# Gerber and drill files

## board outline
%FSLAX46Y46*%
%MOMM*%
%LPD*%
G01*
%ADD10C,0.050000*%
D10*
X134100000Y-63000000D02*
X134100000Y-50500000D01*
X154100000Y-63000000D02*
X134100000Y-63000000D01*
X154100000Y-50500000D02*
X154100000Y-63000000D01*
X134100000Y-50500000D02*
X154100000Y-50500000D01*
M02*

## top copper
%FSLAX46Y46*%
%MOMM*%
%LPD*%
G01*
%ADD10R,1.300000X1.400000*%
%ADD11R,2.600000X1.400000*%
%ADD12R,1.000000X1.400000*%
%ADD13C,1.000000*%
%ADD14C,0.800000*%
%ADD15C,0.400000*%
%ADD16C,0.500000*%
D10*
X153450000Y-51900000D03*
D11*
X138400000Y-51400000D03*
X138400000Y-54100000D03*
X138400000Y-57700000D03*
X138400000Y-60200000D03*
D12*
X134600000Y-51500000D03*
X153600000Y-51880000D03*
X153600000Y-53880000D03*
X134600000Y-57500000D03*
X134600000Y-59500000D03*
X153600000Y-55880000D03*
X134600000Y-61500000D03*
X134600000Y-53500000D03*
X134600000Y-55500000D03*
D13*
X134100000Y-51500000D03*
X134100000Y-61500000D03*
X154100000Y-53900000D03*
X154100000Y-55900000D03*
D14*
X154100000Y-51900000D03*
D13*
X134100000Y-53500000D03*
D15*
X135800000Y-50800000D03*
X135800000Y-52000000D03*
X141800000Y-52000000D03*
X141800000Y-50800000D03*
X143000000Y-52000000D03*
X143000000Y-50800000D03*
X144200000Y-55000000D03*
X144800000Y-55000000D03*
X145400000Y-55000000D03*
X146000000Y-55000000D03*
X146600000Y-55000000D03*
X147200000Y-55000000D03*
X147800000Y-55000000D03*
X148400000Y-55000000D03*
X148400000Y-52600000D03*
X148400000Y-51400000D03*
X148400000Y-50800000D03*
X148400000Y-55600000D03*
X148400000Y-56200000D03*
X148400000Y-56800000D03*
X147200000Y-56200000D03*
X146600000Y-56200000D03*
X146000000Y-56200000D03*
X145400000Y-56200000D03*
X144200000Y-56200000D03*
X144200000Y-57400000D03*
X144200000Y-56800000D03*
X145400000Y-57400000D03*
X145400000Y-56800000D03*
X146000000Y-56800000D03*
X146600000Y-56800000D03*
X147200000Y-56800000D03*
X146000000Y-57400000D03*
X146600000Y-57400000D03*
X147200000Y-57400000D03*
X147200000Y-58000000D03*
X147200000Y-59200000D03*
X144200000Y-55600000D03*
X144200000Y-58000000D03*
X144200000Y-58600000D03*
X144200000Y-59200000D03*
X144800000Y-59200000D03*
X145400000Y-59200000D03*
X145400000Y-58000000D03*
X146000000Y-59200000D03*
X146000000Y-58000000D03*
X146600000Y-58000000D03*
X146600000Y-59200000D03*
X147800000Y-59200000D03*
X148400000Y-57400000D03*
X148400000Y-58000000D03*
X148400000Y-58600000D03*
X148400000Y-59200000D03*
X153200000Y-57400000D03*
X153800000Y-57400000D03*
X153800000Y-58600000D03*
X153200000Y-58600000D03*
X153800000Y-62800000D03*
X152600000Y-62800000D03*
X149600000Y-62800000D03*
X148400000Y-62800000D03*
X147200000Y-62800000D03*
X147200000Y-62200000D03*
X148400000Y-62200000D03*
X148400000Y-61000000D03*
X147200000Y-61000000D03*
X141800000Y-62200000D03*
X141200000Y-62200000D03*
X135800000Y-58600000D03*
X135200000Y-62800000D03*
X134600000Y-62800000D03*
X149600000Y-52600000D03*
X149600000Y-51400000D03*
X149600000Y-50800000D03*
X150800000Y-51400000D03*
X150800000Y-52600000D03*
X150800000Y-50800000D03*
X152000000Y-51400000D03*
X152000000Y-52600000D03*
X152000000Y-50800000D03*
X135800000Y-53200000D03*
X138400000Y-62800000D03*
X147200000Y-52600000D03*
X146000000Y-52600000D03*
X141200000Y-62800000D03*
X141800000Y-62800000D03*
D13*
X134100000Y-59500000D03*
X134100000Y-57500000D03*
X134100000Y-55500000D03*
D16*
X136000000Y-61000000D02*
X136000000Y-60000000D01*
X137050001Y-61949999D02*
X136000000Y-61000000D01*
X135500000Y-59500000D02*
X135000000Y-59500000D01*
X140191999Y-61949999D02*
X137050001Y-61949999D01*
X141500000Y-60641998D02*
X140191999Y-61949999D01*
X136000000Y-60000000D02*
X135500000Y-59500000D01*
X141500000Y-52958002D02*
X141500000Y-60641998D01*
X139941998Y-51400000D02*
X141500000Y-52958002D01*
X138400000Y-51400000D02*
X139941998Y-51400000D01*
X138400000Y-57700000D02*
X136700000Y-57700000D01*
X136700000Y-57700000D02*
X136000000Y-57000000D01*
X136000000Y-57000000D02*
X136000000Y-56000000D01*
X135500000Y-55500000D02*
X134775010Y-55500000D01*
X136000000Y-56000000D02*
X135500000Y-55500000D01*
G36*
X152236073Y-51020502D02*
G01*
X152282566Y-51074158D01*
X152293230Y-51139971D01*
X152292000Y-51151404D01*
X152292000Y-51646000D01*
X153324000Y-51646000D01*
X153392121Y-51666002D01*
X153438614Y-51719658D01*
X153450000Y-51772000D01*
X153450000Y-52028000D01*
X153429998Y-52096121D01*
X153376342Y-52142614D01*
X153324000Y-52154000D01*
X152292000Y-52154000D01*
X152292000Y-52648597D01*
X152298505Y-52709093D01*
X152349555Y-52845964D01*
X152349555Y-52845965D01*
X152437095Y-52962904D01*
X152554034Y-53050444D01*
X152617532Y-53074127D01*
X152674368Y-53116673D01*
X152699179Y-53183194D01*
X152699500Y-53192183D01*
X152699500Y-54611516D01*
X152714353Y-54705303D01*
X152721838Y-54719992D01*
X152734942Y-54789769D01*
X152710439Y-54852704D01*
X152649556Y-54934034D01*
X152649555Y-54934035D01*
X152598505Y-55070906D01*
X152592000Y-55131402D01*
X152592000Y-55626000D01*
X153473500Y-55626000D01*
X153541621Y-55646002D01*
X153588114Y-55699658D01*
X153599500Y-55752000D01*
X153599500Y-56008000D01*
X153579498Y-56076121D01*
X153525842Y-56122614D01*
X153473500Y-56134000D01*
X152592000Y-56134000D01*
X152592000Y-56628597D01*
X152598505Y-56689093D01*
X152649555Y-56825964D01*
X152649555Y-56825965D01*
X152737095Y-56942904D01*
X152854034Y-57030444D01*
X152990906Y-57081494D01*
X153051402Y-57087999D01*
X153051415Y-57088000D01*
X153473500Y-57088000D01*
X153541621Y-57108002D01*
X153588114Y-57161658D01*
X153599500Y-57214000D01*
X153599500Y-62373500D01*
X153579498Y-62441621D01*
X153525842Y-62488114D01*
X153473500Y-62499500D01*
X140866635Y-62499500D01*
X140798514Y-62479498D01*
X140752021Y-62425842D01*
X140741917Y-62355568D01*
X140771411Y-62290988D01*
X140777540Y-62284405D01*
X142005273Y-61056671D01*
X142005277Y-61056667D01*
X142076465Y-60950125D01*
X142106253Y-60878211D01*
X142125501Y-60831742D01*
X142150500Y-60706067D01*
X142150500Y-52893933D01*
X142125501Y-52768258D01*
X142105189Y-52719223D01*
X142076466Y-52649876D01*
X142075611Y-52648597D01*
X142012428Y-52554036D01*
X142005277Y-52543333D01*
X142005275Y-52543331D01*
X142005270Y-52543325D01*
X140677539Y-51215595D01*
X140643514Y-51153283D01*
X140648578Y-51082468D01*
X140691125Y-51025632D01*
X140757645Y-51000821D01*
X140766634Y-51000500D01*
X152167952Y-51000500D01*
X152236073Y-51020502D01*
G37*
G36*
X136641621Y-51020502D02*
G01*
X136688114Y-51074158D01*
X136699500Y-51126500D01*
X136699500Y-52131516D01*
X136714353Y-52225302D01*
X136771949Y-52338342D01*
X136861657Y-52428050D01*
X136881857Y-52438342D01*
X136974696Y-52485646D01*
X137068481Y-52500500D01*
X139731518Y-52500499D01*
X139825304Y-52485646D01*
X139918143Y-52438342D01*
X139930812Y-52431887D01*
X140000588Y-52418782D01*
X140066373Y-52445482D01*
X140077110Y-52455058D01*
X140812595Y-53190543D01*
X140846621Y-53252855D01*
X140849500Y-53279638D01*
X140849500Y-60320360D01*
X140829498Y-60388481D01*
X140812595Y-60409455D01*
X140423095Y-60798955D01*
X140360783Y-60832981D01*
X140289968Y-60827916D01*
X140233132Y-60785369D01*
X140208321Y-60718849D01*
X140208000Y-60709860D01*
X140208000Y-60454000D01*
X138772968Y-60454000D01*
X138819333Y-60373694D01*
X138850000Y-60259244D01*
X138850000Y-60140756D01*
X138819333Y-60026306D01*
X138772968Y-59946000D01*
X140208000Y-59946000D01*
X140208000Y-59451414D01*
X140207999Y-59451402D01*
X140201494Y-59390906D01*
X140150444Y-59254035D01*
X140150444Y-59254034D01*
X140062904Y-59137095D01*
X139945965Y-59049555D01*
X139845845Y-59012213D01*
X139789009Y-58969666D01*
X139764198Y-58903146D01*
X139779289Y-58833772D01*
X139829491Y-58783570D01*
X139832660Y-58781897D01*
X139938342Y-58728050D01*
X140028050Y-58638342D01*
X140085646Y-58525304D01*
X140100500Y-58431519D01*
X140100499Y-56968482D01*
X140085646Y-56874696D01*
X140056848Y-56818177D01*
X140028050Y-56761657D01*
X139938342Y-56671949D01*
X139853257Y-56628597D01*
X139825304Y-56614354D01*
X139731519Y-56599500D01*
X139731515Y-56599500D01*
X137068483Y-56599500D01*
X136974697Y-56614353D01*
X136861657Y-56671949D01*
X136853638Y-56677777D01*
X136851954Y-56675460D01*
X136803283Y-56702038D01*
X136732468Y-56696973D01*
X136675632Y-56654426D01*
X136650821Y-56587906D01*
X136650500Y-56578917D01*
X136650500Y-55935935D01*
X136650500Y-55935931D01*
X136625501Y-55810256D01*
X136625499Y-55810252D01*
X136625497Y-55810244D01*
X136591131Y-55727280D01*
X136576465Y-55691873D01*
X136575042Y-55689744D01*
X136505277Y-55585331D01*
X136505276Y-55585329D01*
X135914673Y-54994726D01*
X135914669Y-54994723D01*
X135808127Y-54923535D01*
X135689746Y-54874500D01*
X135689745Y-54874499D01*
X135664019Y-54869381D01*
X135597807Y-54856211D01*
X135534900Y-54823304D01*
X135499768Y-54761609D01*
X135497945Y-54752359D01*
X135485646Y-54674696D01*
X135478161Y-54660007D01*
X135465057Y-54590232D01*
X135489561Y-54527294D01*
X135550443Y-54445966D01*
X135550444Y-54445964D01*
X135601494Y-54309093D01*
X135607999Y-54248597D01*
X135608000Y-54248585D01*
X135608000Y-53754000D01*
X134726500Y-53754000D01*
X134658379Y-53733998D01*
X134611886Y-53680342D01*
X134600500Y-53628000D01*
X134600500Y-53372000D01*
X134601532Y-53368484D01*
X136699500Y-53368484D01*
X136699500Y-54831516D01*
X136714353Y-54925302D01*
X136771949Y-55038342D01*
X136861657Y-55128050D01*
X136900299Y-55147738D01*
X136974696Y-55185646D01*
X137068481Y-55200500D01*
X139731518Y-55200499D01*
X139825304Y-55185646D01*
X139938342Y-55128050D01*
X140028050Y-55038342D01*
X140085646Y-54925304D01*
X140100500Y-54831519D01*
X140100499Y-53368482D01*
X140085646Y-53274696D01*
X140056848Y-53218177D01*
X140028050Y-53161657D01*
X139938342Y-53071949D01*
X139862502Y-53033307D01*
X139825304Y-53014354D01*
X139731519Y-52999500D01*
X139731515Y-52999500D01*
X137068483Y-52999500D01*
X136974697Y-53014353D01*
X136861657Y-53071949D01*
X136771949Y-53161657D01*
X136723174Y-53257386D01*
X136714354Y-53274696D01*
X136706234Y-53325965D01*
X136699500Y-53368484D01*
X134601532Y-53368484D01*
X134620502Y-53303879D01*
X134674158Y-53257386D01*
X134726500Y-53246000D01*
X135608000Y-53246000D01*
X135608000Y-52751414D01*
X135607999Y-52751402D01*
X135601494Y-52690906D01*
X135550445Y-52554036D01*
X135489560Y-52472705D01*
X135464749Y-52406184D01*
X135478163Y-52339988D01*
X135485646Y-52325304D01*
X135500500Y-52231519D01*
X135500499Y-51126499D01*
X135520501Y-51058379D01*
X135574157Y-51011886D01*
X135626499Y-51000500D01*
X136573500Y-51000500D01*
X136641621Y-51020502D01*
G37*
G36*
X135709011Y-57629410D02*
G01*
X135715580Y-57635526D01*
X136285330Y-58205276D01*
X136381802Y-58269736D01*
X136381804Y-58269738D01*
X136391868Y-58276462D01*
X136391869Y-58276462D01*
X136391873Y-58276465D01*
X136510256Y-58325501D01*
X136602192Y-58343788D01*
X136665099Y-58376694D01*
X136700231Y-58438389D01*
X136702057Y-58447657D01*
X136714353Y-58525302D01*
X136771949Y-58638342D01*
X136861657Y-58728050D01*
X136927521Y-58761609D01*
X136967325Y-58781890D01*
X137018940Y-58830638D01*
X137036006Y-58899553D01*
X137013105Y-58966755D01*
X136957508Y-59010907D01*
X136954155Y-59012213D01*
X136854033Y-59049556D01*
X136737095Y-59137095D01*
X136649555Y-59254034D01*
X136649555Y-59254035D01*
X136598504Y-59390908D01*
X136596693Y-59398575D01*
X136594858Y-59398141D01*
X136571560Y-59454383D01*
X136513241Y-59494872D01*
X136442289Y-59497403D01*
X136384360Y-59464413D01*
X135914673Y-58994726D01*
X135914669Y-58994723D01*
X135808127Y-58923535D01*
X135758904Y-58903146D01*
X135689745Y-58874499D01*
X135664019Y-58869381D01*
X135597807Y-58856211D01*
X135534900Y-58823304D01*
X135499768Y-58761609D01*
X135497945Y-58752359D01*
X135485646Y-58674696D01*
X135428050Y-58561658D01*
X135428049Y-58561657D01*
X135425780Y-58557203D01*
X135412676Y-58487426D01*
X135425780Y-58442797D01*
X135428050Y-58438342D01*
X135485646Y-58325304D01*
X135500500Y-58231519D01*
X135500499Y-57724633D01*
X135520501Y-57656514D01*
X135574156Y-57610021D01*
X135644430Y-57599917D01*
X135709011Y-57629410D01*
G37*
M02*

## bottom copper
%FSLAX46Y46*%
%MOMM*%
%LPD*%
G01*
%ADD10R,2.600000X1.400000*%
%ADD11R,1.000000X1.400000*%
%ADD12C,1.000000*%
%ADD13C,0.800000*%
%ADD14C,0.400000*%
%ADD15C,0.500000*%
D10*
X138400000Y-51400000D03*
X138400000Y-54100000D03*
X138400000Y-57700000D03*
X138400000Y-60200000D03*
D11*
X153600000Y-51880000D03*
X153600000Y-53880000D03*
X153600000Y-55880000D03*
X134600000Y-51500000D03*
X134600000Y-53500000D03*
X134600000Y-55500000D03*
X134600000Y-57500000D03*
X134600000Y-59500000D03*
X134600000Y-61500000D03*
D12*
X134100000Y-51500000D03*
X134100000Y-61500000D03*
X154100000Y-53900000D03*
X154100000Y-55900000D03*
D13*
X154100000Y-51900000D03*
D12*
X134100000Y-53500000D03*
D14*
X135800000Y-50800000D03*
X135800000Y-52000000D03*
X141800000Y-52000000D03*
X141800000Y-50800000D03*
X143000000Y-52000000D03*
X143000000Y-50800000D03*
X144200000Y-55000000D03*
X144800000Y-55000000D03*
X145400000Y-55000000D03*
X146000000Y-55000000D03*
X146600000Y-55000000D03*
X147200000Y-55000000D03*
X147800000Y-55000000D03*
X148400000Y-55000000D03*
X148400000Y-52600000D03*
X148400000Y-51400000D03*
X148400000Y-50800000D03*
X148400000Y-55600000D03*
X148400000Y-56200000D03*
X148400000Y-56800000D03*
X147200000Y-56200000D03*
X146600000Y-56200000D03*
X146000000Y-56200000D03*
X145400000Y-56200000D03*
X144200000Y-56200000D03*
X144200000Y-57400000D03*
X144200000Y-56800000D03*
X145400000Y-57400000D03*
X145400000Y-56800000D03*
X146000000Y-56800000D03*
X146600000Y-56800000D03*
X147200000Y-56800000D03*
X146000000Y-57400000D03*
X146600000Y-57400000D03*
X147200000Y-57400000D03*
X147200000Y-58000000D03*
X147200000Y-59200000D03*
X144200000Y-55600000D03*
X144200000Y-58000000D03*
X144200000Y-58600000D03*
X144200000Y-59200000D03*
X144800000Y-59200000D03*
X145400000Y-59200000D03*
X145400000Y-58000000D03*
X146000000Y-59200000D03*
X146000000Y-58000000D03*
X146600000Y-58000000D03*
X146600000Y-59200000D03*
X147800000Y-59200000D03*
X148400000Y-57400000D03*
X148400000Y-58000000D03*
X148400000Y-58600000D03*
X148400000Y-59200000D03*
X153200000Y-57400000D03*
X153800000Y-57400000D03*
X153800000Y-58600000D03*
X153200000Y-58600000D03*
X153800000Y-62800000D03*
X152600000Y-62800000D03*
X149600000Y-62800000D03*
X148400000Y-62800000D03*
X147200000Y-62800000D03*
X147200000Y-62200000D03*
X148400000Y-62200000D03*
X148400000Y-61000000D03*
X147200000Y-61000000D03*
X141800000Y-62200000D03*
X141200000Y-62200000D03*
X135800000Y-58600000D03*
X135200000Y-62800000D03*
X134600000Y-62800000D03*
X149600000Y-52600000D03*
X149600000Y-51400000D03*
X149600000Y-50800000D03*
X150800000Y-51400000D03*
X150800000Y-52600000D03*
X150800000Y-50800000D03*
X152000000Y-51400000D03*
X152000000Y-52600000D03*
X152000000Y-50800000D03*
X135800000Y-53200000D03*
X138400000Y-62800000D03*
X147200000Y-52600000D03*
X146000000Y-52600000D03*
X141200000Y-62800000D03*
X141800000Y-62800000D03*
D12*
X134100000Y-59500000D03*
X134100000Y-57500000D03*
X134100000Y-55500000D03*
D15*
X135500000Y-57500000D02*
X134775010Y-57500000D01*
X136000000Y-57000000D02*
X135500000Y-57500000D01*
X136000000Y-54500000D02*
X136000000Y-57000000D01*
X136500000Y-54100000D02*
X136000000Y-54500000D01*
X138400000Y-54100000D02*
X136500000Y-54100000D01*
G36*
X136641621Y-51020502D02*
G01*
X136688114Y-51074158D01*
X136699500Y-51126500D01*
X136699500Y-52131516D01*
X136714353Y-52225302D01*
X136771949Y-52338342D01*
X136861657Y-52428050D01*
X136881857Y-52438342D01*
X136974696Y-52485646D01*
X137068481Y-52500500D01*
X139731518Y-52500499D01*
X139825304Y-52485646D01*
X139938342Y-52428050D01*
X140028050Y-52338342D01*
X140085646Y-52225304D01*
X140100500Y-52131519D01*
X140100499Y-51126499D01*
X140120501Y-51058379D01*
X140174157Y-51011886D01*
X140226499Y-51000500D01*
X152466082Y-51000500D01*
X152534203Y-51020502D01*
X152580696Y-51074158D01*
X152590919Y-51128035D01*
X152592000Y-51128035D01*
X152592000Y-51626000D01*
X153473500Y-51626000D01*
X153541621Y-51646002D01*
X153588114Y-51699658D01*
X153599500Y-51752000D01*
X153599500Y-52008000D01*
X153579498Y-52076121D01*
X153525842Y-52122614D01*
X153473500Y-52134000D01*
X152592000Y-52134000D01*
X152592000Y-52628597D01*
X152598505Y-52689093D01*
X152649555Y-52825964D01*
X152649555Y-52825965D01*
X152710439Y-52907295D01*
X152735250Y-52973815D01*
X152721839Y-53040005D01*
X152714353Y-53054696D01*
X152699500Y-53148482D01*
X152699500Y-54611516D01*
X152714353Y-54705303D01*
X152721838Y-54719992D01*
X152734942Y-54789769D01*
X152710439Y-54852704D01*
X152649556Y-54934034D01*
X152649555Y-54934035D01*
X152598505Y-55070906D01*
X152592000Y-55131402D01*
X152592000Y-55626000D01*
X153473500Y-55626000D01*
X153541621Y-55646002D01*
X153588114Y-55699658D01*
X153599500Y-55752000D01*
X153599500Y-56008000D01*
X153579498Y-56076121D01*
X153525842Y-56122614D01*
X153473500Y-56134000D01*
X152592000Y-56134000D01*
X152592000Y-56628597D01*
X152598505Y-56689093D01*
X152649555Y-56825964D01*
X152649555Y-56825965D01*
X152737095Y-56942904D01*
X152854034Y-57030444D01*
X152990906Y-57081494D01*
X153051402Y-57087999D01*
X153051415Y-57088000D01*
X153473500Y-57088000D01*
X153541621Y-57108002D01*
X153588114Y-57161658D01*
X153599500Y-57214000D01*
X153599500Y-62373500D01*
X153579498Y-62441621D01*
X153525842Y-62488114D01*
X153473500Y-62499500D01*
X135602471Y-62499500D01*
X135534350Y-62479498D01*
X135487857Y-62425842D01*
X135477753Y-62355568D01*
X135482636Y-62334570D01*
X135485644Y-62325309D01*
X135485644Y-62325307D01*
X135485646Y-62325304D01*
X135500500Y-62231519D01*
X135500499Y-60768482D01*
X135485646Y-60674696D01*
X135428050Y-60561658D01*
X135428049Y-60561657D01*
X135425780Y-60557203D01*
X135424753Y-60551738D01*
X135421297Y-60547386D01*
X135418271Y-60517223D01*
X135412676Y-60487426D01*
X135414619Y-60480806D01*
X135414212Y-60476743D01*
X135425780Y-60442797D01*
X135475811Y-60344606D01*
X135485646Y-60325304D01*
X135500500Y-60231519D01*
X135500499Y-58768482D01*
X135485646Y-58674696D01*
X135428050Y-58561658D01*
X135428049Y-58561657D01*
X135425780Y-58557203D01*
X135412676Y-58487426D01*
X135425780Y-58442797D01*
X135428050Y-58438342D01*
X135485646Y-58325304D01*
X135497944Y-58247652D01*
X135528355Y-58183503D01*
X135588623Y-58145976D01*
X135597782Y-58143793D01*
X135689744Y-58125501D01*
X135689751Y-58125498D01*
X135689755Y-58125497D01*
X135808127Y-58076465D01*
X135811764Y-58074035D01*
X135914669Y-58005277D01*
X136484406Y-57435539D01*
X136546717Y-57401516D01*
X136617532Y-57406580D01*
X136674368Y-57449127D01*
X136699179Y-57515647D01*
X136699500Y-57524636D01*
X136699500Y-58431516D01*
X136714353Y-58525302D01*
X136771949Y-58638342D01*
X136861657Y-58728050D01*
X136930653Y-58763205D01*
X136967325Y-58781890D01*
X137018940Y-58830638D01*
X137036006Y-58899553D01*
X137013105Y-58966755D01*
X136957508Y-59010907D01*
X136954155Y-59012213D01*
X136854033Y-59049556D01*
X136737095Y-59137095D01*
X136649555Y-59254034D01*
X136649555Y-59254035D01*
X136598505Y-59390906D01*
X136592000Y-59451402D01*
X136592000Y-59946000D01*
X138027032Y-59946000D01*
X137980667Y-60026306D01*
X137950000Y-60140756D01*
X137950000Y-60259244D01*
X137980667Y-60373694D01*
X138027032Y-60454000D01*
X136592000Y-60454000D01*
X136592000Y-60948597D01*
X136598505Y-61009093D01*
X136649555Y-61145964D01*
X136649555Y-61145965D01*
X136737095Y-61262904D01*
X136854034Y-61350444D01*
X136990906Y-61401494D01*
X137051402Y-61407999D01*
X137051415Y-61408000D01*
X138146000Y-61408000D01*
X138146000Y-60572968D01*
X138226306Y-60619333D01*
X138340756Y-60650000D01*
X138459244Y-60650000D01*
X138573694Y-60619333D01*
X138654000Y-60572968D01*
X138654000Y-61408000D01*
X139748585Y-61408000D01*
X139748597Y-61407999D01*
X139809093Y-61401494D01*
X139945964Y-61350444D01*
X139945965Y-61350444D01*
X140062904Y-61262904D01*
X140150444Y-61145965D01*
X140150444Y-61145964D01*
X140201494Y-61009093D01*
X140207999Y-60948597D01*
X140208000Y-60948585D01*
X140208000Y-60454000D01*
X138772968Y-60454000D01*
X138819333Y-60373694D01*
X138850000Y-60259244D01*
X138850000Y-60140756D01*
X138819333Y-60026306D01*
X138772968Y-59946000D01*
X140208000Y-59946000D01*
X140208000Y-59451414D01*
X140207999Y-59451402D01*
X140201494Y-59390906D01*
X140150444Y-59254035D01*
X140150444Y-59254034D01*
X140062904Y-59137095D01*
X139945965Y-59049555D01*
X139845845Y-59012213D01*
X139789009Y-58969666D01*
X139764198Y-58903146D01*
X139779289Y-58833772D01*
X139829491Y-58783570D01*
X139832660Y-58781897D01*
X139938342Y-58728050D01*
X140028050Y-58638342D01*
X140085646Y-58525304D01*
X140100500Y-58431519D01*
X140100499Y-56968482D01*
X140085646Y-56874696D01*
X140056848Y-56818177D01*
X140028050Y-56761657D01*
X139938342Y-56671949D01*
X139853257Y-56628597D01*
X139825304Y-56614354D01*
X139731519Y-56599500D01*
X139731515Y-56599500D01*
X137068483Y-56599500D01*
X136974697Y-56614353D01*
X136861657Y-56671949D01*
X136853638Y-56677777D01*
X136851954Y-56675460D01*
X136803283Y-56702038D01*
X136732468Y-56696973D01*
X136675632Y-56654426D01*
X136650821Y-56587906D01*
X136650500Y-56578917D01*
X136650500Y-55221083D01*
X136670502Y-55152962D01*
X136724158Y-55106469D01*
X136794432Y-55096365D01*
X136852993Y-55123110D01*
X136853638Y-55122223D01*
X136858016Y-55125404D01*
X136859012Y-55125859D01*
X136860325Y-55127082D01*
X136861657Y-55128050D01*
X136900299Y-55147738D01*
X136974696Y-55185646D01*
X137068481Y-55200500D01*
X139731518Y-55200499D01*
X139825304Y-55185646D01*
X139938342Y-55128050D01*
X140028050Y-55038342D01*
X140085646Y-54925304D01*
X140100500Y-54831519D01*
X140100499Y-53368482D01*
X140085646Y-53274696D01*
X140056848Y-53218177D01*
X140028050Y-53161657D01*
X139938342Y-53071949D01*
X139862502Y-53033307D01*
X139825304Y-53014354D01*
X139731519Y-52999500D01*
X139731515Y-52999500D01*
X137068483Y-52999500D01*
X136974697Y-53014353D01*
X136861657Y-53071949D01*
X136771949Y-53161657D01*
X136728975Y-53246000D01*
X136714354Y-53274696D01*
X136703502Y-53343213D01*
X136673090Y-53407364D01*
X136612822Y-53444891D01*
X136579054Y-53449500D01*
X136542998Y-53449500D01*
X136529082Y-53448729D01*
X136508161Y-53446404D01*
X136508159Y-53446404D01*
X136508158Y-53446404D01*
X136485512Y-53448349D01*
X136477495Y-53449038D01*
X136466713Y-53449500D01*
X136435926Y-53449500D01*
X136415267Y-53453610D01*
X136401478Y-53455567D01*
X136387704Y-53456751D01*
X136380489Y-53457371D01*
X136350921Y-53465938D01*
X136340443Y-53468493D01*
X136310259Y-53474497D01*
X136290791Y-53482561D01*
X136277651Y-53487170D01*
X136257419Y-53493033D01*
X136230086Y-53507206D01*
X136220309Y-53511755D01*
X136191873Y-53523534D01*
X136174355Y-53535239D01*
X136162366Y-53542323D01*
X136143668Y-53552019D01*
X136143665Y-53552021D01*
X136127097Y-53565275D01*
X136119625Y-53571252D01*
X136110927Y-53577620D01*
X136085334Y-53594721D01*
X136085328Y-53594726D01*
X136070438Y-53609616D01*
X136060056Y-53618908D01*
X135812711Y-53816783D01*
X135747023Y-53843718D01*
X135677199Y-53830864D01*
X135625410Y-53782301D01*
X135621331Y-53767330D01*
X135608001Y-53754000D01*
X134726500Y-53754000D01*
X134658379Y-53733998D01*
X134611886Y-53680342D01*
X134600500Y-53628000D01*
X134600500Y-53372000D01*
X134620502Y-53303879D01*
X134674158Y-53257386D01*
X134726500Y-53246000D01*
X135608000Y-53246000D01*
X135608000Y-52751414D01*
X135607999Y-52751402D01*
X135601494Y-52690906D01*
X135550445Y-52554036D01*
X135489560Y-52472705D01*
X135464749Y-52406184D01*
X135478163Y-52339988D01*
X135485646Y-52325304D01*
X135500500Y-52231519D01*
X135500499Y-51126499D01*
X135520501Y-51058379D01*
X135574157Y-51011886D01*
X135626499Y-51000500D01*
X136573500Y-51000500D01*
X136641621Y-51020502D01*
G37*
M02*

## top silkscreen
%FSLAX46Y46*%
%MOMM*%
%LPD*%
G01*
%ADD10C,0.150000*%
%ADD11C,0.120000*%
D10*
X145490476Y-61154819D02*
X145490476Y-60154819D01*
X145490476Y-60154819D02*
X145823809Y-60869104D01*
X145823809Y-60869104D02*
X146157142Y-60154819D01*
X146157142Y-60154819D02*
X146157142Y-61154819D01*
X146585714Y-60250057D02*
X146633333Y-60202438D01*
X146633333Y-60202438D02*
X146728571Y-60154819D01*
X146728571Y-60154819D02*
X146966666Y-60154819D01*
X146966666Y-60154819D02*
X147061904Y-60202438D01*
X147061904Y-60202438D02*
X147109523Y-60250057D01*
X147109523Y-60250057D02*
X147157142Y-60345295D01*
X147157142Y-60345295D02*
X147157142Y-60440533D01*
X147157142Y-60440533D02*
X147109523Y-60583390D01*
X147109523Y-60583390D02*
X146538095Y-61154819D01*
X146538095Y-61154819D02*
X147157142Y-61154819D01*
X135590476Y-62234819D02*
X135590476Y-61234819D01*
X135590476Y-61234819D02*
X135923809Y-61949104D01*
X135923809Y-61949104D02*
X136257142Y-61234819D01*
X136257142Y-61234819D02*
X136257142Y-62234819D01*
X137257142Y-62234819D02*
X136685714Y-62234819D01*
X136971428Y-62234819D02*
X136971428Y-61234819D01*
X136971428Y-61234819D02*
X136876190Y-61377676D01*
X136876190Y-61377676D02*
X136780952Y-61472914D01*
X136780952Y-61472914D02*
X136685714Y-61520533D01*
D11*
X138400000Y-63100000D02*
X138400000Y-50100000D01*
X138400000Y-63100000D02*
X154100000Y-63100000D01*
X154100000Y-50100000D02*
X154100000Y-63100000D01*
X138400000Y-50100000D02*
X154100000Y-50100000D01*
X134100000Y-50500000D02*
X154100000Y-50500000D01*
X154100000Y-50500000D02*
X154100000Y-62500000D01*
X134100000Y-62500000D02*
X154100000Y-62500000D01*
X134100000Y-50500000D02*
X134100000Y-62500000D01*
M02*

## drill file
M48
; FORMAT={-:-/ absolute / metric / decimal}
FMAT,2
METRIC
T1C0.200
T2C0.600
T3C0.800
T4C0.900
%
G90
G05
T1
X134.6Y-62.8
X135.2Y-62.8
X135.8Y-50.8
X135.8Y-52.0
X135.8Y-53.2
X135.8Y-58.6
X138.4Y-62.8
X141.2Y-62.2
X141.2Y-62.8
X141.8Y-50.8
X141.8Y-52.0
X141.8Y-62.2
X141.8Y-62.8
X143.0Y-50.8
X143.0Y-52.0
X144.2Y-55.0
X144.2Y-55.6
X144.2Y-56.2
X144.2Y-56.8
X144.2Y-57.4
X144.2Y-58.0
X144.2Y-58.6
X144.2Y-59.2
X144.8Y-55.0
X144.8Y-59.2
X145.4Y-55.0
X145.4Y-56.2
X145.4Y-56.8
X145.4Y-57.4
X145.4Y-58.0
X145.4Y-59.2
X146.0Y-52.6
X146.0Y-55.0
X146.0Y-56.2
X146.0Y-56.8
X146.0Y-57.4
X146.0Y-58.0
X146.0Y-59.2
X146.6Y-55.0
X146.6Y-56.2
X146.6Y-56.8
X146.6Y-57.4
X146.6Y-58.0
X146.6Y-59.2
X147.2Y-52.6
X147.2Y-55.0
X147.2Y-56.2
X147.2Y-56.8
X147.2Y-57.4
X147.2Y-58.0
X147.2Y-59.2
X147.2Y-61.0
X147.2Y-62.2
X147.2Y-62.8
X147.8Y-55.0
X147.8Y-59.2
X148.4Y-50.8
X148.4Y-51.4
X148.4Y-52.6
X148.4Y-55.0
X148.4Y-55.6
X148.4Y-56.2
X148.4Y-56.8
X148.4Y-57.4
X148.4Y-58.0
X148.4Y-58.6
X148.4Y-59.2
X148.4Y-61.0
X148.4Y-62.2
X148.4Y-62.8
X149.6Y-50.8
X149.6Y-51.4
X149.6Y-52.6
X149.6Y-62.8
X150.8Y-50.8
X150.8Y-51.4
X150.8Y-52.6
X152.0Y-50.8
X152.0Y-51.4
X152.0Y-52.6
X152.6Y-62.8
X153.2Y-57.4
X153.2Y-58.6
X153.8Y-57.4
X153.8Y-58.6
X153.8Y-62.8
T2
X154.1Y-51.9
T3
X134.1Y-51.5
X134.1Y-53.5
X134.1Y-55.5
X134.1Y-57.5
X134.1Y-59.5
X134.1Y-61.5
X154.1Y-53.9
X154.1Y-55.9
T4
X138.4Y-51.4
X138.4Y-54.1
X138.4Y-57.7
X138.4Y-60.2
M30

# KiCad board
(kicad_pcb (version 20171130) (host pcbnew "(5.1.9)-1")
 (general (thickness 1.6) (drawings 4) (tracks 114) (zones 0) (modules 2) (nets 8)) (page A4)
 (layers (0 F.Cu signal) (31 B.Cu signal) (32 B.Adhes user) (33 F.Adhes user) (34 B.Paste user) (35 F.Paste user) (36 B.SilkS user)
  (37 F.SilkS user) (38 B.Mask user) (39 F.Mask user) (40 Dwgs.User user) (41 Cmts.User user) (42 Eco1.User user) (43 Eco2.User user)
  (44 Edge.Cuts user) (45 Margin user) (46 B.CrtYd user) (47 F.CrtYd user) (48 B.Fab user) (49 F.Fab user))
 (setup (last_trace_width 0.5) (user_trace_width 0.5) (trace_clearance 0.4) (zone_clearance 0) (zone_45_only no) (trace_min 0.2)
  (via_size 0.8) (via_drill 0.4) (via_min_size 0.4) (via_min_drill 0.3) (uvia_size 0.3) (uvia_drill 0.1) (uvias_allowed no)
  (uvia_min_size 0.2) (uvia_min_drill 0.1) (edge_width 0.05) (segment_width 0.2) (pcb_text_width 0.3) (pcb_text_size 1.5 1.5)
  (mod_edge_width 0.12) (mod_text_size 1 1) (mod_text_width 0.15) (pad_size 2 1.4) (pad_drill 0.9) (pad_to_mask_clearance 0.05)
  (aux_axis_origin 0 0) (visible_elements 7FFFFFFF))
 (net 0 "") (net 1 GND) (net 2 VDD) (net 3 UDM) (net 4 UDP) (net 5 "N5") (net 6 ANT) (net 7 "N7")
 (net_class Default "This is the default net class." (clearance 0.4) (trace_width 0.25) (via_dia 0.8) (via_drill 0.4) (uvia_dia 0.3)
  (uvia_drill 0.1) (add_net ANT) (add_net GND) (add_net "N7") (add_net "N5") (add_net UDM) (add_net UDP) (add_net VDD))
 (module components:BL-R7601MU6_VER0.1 (layer F.Cu) (at 138.4 50.1)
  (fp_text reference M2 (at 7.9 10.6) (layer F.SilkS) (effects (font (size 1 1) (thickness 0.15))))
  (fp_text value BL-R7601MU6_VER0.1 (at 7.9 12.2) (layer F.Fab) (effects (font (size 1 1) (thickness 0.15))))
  (fp_line (start 0 13) (end 0 0) (layer F.SilkS) (width 0.12))
  (fp_line (start 0 13) (end 15.7 13) (layer F.SilkS) (width 0.12))
  (fp_line (start 15.7 0) (end 15.7 13) (layer F.SilkS) (width 0.12))
  (fp_line (start 0 0) (end 15.7 0) (layer F.SilkS) (width 0.12))
  (pad 5 smd rect (at 15.7 1.8) (size 1.3 1.4) (drill (offset -0.65 0)) (layers F.Cu F.Paste F.Mask) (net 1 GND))
  (pad 4 thru_hole rect (at 0 1.3) (size 2.6 1.4) (drill 0.9) (layers *.Cu *.Mask) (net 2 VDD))
  (pad 3 thru_hole rect (at 0 4) (size 2.6 1.4) (drill 0.9) (layers *.Cu *.Mask) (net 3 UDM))
  (pad 2 thru_hole rect (at 0 7.6) (size 2.6 1.4) (drill 0.9) (layers *.Cu *.Mask) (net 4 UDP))
  (pad 1 thru_hole rect (at 0 10.1) (size 2.6 1.4) (drill 0.9) (layers *.Cu *.Mask) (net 1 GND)))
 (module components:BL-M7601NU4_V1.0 (layer F.Cu) (at 134.1 50.5)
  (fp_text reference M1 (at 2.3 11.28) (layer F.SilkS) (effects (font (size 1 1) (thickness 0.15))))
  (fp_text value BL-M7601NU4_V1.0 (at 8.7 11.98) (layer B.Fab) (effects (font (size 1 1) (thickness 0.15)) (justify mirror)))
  (fp_line (start 0 0) (end 20 0) (layer F.SilkS) (width 0.12))
  (fp_line (start 20 0) (end 20 12) (layer F.SilkS) (width 0.12))
  (fp_line (start 0 12) (end 20 12) (layer F.SilkS) (width 0.12))
  (fp_line (start 0 0) (end 0 12) (layer F.SilkS) (width 0.12))
  (pad 6 smd rect (at 0 1) (size 1 1.4) (drill (offset 0.5 0)) (layers F.Cu F.Paste F.Mask) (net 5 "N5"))
  (pad 9 smd rect (at 20 1.38) (size 1 1.4) (drill (offset -0.5 0)) (layers F.Cu F.Paste F.Mask) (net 1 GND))
  (pad 8 smd rect (at 20 3.38) (size 1 1.4) (drill (offset -0.5 0)) (layers F.Cu F.Paste F.Mask) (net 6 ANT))
  (pad 3 smd rect (at 0 7) (size 1 1.4) (drill (offset 0.5 0)) (layers F.Cu F.Paste F.Mask) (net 3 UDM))
  (pad 2 smd rect (at 0 9) (size 1 1.4) (drill (offset 0.5 0)) (layers F.Cu F.Paste F.Mask) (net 2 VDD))
  (pad 7 smd rect (at 20 5.38) (size 1 1.4) (drill (offset -0.5 0)) (layers F.Cu F.Paste F.Mask) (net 1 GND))
  (pad 1 smd rect (at 0 11) (size 1 1.4) (drill (offset 0.5 0)) (layers F.Cu F.Paste F.Mask) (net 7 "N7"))
  (pad 5 smd rect (at 0 3) (size 1 1.4) (drill (offset 0.5 0)) (layers F.Cu F.Paste F.Mask) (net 1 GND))
  (pad 4 smd rect (at 0 5) (size 1 1.4) (drill (offset 0.5 0)) (layers F.Cu F.Paste F.Mask) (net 4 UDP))
  (pad 9 smd rect (at 20 1.38) (size 1 1.4) (drill (offset -0.5 0)) (layers B.Cu B.Paste B.Mask) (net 1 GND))
  (pad 8 smd rect (at 20 3.38) (size 1 1.4) (drill (offset -0.5 0)) (layers B.Cu B.Paste B.Mask) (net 6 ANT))
  (pad 7 smd rect (at 20 5.38) (size 1 1.4) (drill (offset -0.5 0)) (layers B.Cu B.Paste B.Mask) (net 1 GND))
  (pad 6 smd rect (at 0 1) (size 1 1.4) (drill (offset 0.5 0)) (layers B.Cu B.Paste B.Mask) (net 5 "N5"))
  (pad 5 smd rect (at 0 3) (size 1 1.4) (drill (offset 0.5 0)) (layers B.Cu B.Paste B.Mask) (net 1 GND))
  (pad 4 smd rect (at 0 5) (size 1 1.4) (drill (offset 0.5 0)) (layers B.Cu B.Paste B.Mask) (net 4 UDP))
  (pad 3 smd rect (at 0 7) (size 1 1.4) (drill (offset 0.5 0)) (layers B.Cu B.Paste B.Mask) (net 3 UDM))
  (pad 2 smd rect (at 0 9) (size 1 1.4) (drill (offset 0.5 0)) (layers B.Cu B.Paste B.Mask) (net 2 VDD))
  (pad 1 smd rect (at 0 11) (size 1 1.4) (drill (offset 0.5 0)) (layers B.Cu B.Paste B.Mask) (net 7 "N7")))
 (gr_line (start 134.1 63) (end 134.1 50.5) (layer Edge.Cuts) (width 0.05))
 (gr_line (start 154.1 63) (end 134.1 63) (layer Edge.Cuts) (width 0.05))
 (gr_line (start 154.1 50.5) (end 154.1 63) (layer Edge.Cuts) (width 0.05))
 (gr_line (start 134.1 50.5) (end 154.1 50.5) (layer Edge.Cuts) (width 0.05))
 (via (at 134.1 51.5) (size 1) (drill 0.8) (layers F.Cu B.Cu) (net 5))
 (via (at 134.1 61.5) (size 1) (drill 0.8) (layers F.Cu B.Cu) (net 7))
 (via (at 154.1 53.9) (size 1) (drill 0.8) (layers F.Cu B.Cu) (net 6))
 (via (at 154.1 55.9) (size 1) (drill 0.8) (layers F.Cu B.Cu) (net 1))
 (via (at 154.1 51.9) (size 0.8) (drill 0.6) (layers F.Cu B.Cu) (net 1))
 (via (at 134.1 53.5) (size 1) (drill 0.8) (layers F.Cu B.Cu) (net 1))
 (via (at 135.8 50.8) (size 0.4) (drill 0.2) (layers F.Cu B.Cu) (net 1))
 (via (at 135.8 52) (size 0.4) (drill 0.2) (layers F.Cu B.Cu) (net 1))
 (via (at 141.8 52) (size 0.4) (drill 0.2) (layers F.Cu B.Cu) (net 1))
 (via (at 141.8 50.8) (size 0.4) (drill 0.2) (layers F.Cu B.Cu) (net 1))
 (via (at 143 52) (size 0.4) (drill 0.2) (layers F.Cu B.Cu) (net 1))
 (via (at 143 50.8) (size 0.4) (drill 0.2) (layers F.Cu B.Cu) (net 1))
 (via (at 144.2 55) (size 0.4) (drill 0.2) (layers F.Cu B.Cu) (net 1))
 (via (at 144.8 55) (size 0.4) (drill 0.2) (layers F.Cu B.Cu) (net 1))
 (via (at 145.4 55) (size 0.4) (drill 0.2) (layers F.Cu B.Cu) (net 1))
 (via (at 146 55) (size 0.4) (drill 0.2) (layers F.Cu B.Cu) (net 1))
 (via (at 146.6 55) (size 0.4) (drill 0.2) (layers F.Cu B.Cu) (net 1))
 (via (at 147.2 55) (size 0.4) (drill 0.2) (layers F.Cu B.Cu) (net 1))
 (via (at 147.8 55) (size 0.4) (drill 0.2) (layers F.Cu B.Cu) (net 1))
 (via (at 148.4 55) (size 0.4) (drill 0.2) (layers F.Cu B.Cu) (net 1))
 (via (at 148.4 52.6) (size 0.4) (drill 0.2) (layers F.Cu B.Cu) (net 1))
 (via (at 148.4 51.4) (size 0.4) (drill 0.2) (layers F.Cu B.Cu) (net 1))
 (via (at 148.4 50.8) (size 0.4) (drill 0.2) (layers F.Cu B.Cu) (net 1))
 (via (at 148.4 55.6) (size 0.4) (drill 0.2) (layers F.Cu B.Cu) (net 1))
 (via (at 148.4 56.2) (size 0.4) (drill 0.2) (layers F.Cu B.Cu) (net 1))
 (via (at 148.4 56.8) (size 0.4) (drill 0.2) (layers F.Cu B.Cu) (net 1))
 (via (at 147.2 56.2) (size 0.4) (drill 0.2) (layers F.Cu B.Cu) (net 1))
 (via (at 146.6 56.2) (size 0.4) (drill 0.2) (layers F.Cu B.Cu) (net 1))
 (via (at 146 56.2) (size 0.4) (drill 0.2) (layers F.Cu B.Cu) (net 1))
 (via (at 145.4 56.2) (size 0.4) (drill 0.2) (layers F.Cu B.Cu) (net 1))
 (via (at 144.2 56.2) (size 0.4) (drill 0.2) (layers F.Cu B.Cu) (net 1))
 (via (at 144.2 57.4) (size 0.4) (drill 0.2) (layers F.Cu B.Cu) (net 1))
 (via (at 144.2 56.8) (size 0.4) (drill 0.2) (layers F.Cu B.Cu) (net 1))
 (via (at 145.4 57.4) (size 0.4) (drill 0.2) (layers F.Cu B.Cu) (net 1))
 (via (at 145.4 56.8) (size 0.4) (drill 0.2) (layers F.Cu B.Cu) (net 1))
 (via (at 146 56.8) (size 0.4) (drill 0.2) (layers F.Cu B.Cu) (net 1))
 (via (at 146.6 56.8) (size 0.4) (drill 0.2) (layers F.Cu B.Cu) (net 1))
 (via (at 147.2 56.8) (size 0.4) (drill 0.2) (layers F.Cu B.Cu) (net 1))
 (via (at 146 57.4) (size 0.4) (drill 0.2) (layers F.Cu B.Cu) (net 1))
 (via (at 146.6 57.4) (size 0.4) (drill 0.2) (layers F.Cu B.Cu) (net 1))
 (via (at 147.2 57.4) (size 0.4) (drill 0.2) (layers F.Cu B.Cu) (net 1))
 (via (at 147.2 58) (size 0.4) (drill 0.2) (layers F.Cu B.Cu) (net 1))
 (via (at 147.2 59.2) (size 0.4) (drill 0.2) (layers F.Cu B.Cu) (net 1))
 (via (at 144.2 55.6) (size 0.4) (drill 0.2) (layers F.Cu B.Cu) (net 1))
 (via (at 144.2 58) (size 0.4) (drill 0.2) (layers F.Cu B.Cu) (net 1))
 (via (at 144.2 58.6) (size 0.4) (drill 0.2) (layers F.Cu B.Cu) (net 1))
 (via (at 144.2 59.2) (size 0.4) (drill 0.2) (layers F.Cu B.Cu) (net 1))
 (via (at 144.8 59.2) (size 0.4) (drill 0.2) (layers F.Cu B.Cu) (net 1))
 (via (at 145.4 59.2) (size 0.4) (drill 0.2) (layers F.Cu B.Cu) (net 1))
 (via (at 145.4 58) (size 0.4) (drill 0.2) (layers F.Cu B.Cu) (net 1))
 (via (at 146 59.2) (size 0.4) (drill 0.2) (layers F.Cu B.Cu) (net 1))
 (via (at 146 58) (size 0.4) (drill 0.2) (layers F.Cu B.Cu) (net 1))
 (via (at 146.6 58) (size 0.4) (drill 0.2) (layers F.Cu B.Cu) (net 1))
 (via (at 146.6 59.2) (size 0.4) (drill 0.2) (layers F.Cu B.Cu) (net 1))
 (via (at 147.8 59.2) (size 0.4) (drill 0.2) (layers F.Cu B.Cu) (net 1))
 (via (at 148.4 57.4) (size 0.4) (drill 0.2) (layers F.Cu B.Cu) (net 1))
 (via (at 148.4 58) (size 0.4) (drill 0.2) (layers F.Cu B.Cu) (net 1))
 (via (at 148.4 58.6) (size 0.4) (drill 0.2) (layers F.Cu B.Cu) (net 1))
 (via (at 148.4 59.2) (size 0.4) (drill 0.2) (layers F.Cu B.Cu) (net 1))
 (via (at 153.2 57.4) (size 0.4) (drill 0.2) (layers F.Cu B.Cu) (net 1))
 (via (at 153.8 57.4) (size 0.4) (drill 0.2) (layers F.Cu B.Cu) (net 1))
 (via (at 153.8 58.6) (size 0.4) (drill 0.2) (layers F.Cu B.Cu) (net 1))
 (via (at 153.2 58.6) (size 0.4) (drill 0.2) (layers F.Cu B.Cu) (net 1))
 (via (at 153.8 62.8) (size 0.4) (drill 0.2) (layers F.Cu B.Cu) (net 1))
 (via (at 152.6 62.8) (size 0.4) (drill 0.2) (layers F.Cu B.Cu) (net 1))
 (via (at 149.6 62.8) (size 0.4) (drill 0.2) (layers F.Cu B.Cu) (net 1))
 (via (at 148.4 62.8) (size 0.4) (drill 0.2) (layers F.Cu B.Cu) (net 1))
 (via (at 147.2 62.8) (size 0.4) (drill 0.2) (layers F.Cu B.Cu) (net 1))
 (via (at 147.2 62.2) (size 0.4) (drill 0.2) (layers F.Cu B.Cu) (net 1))
 (via (at 148.4 62.2) (size 0.4) (drill 0.2) (layers F.Cu B.Cu) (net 1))
 (via (at 148.4 61) (size 0.4) (drill 0.2) (layers F.Cu B.Cu) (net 1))
 (via (at 147.2 61) (size 0.4) (drill 0.2) (layers F.Cu B.Cu) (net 1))
 (via (at 141.8 62.2) (size 0.4) (drill 0.2) (layers F.Cu B.Cu) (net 1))
 (via (at 141.2 62.2) (size 0.4) (drill 0.2) (layers F.Cu B.Cu) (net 1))
 (via (at 135.8 58.6) (size 0.4) (drill 0.2) (layers F.Cu B.Cu) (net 1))
 (via (at 135.2 62.8) (size 0.4) (drill 0.2) (layers F.Cu B.Cu) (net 1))
 (via (at 134.6 62.8) (size 0.4) (drill 0.2) (layers F.Cu B.Cu) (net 1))
 (via (at 149.6 52.6) (size 0.4) (drill 0.2) (layers F.Cu B.Cu) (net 1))
 (via (at 149.6 51.4) (size 0.4) (drill 0.2) (layers F.Cu B.Cu) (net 1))
 (via (at 149.6 50.8) (size 0.4) (drill 0.2) (layers F.Cu B.Cu) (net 1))
 (via (at 150.8 51.4) (size 0.4) (drill 0.2) (layers F.Cu B.Cu) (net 1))
 (via (at 150.8 52.6) (size 0.4) (drill 0.2) (layers F.Cu B.Cu) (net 1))
 (via (at 150.8 50.8) (size 0.4) (drill 0.2) (layers F.Cu B.Cu) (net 1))
 (via (at 152 51.4) (size 0.4) (drill 0.2) (layers F.Cu B.Cu) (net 1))
 (via (at 152 52.6) (size 0.4) (drill 0.2) (layers F.Cu B.Cu) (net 1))
 (via (at 152 50.8) (size 0.4) (drill 0.2) (layers F.Cu B.Cu) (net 1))
 (via (at 135.8 53.2) (size 0.4) (drill 0.2) (layers F.Cu B.Cu) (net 1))
 (via (at 138.4 62.8) (size 0.4) (drill 0.2) (layers F.Cu B.Cu) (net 1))
 (via (at 147.2 52.6) (size 0.4) (drill 0.2) (layers F.Cu B.Cu) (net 1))
 (via (at 146 52.6) (size 0.4) (drill 0.2) (layers F.Cu B.Cu) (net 1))
 (via (at 141.2 62.8) (size 0.4) (drill 0.2) (layers F.Cu B.Cu) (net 1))
 (via (at 141.8 62.8) (size 0.4) (drill 0.2) (layers F.Cu B.Cu) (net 1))
 (via (at 134.1 59.5) (size 1) (drill 0.8) (layers F.Cu B.Cu) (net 2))
 (segment (start 136 61) (end 136 60) (width 0.5) (layer F.Cu) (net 2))
 (segment (start 137.050001 61.949999) (end 136 61) (width 0.5) (layer F.Cu) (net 2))
 (segment (start 135.5 59.5) (end 135 59.5) (width 0.5) (layer F.Cu) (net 2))
 (segment (start 140.191999 61.949999) (end 137.050001 61.949999) (width 0.5) (layer F.Cu) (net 2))
 (segment (start 141.5 60.641998) (end 140.191999 61.949999) (width 0.5) (layer F.Cu) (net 2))
 (segment (start 136 60) (end 135.5 59.5) (width 0.5) (layer F.Cu) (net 2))
 (segment (start 141.5 52.958002) (end 141.5 60.641998) (width 0.5) (layer F.Cu) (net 2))
 (segment (start 139.941998 51.4) (end 141.5 52.958002) (width 0.5) (layer F.Cu) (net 2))
 (segment (start 138.4 51.4) (end 139.941998 51.4) (width 0.5) (layer F.Cu) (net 2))
 (via (at 134.1 57.5) (size 1) (drill 0.8) (layers F.Cu B.Cu) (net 3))
 (segment (start 135.5 57.5) (end 134.77501 57.5) (width 0.5) (layer B.Cu) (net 3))
 (segment (start 136 57) (end 135.5 57.5) (width 0.5) (layer B.Cu) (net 3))
 (segment (start 136 54.5) (end 136 57) (width 0.5) (layer B.Cu) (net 3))
 (segment (start 136.5 54.1) (end 136 54.5) (width 0.5) (layer B.Cu) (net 3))
 (segment (start 138.4 54.1) (end 136.5 54.1) (width 0.5) (layer B.Cu) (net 3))
 (via (at 134.1 55.5) (size 1) (drill 0.8) (layers F.Cu B.Cu) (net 4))
 (segment (start 138.4 57.7) (end 136.7 57.7) (width 0.5) (layer F.Cu) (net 4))
 (segment (start 136.7 57.7) (end 136 57) (width 0.5) (layer F.Cu) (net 4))
 (segment (start 136 57) (end 136 56) (width 0.5) (layer F.Cu) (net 4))
 (segment (start 135.5 55.5) (end 134.77501 55.5) (width 0.5) (layer F.Cu) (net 4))
 (segment (start 136 56) (end 135.5 55.5) (width 0.5) (layer F.Cu) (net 4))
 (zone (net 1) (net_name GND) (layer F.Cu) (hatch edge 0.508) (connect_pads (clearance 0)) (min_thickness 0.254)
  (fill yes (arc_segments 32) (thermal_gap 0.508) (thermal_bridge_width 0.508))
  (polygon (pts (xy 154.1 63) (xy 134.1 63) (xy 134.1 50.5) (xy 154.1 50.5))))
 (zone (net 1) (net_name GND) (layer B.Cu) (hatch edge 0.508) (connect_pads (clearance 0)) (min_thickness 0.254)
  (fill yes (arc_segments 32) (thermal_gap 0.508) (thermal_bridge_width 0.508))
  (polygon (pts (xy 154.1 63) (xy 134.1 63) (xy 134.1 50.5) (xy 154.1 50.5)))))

